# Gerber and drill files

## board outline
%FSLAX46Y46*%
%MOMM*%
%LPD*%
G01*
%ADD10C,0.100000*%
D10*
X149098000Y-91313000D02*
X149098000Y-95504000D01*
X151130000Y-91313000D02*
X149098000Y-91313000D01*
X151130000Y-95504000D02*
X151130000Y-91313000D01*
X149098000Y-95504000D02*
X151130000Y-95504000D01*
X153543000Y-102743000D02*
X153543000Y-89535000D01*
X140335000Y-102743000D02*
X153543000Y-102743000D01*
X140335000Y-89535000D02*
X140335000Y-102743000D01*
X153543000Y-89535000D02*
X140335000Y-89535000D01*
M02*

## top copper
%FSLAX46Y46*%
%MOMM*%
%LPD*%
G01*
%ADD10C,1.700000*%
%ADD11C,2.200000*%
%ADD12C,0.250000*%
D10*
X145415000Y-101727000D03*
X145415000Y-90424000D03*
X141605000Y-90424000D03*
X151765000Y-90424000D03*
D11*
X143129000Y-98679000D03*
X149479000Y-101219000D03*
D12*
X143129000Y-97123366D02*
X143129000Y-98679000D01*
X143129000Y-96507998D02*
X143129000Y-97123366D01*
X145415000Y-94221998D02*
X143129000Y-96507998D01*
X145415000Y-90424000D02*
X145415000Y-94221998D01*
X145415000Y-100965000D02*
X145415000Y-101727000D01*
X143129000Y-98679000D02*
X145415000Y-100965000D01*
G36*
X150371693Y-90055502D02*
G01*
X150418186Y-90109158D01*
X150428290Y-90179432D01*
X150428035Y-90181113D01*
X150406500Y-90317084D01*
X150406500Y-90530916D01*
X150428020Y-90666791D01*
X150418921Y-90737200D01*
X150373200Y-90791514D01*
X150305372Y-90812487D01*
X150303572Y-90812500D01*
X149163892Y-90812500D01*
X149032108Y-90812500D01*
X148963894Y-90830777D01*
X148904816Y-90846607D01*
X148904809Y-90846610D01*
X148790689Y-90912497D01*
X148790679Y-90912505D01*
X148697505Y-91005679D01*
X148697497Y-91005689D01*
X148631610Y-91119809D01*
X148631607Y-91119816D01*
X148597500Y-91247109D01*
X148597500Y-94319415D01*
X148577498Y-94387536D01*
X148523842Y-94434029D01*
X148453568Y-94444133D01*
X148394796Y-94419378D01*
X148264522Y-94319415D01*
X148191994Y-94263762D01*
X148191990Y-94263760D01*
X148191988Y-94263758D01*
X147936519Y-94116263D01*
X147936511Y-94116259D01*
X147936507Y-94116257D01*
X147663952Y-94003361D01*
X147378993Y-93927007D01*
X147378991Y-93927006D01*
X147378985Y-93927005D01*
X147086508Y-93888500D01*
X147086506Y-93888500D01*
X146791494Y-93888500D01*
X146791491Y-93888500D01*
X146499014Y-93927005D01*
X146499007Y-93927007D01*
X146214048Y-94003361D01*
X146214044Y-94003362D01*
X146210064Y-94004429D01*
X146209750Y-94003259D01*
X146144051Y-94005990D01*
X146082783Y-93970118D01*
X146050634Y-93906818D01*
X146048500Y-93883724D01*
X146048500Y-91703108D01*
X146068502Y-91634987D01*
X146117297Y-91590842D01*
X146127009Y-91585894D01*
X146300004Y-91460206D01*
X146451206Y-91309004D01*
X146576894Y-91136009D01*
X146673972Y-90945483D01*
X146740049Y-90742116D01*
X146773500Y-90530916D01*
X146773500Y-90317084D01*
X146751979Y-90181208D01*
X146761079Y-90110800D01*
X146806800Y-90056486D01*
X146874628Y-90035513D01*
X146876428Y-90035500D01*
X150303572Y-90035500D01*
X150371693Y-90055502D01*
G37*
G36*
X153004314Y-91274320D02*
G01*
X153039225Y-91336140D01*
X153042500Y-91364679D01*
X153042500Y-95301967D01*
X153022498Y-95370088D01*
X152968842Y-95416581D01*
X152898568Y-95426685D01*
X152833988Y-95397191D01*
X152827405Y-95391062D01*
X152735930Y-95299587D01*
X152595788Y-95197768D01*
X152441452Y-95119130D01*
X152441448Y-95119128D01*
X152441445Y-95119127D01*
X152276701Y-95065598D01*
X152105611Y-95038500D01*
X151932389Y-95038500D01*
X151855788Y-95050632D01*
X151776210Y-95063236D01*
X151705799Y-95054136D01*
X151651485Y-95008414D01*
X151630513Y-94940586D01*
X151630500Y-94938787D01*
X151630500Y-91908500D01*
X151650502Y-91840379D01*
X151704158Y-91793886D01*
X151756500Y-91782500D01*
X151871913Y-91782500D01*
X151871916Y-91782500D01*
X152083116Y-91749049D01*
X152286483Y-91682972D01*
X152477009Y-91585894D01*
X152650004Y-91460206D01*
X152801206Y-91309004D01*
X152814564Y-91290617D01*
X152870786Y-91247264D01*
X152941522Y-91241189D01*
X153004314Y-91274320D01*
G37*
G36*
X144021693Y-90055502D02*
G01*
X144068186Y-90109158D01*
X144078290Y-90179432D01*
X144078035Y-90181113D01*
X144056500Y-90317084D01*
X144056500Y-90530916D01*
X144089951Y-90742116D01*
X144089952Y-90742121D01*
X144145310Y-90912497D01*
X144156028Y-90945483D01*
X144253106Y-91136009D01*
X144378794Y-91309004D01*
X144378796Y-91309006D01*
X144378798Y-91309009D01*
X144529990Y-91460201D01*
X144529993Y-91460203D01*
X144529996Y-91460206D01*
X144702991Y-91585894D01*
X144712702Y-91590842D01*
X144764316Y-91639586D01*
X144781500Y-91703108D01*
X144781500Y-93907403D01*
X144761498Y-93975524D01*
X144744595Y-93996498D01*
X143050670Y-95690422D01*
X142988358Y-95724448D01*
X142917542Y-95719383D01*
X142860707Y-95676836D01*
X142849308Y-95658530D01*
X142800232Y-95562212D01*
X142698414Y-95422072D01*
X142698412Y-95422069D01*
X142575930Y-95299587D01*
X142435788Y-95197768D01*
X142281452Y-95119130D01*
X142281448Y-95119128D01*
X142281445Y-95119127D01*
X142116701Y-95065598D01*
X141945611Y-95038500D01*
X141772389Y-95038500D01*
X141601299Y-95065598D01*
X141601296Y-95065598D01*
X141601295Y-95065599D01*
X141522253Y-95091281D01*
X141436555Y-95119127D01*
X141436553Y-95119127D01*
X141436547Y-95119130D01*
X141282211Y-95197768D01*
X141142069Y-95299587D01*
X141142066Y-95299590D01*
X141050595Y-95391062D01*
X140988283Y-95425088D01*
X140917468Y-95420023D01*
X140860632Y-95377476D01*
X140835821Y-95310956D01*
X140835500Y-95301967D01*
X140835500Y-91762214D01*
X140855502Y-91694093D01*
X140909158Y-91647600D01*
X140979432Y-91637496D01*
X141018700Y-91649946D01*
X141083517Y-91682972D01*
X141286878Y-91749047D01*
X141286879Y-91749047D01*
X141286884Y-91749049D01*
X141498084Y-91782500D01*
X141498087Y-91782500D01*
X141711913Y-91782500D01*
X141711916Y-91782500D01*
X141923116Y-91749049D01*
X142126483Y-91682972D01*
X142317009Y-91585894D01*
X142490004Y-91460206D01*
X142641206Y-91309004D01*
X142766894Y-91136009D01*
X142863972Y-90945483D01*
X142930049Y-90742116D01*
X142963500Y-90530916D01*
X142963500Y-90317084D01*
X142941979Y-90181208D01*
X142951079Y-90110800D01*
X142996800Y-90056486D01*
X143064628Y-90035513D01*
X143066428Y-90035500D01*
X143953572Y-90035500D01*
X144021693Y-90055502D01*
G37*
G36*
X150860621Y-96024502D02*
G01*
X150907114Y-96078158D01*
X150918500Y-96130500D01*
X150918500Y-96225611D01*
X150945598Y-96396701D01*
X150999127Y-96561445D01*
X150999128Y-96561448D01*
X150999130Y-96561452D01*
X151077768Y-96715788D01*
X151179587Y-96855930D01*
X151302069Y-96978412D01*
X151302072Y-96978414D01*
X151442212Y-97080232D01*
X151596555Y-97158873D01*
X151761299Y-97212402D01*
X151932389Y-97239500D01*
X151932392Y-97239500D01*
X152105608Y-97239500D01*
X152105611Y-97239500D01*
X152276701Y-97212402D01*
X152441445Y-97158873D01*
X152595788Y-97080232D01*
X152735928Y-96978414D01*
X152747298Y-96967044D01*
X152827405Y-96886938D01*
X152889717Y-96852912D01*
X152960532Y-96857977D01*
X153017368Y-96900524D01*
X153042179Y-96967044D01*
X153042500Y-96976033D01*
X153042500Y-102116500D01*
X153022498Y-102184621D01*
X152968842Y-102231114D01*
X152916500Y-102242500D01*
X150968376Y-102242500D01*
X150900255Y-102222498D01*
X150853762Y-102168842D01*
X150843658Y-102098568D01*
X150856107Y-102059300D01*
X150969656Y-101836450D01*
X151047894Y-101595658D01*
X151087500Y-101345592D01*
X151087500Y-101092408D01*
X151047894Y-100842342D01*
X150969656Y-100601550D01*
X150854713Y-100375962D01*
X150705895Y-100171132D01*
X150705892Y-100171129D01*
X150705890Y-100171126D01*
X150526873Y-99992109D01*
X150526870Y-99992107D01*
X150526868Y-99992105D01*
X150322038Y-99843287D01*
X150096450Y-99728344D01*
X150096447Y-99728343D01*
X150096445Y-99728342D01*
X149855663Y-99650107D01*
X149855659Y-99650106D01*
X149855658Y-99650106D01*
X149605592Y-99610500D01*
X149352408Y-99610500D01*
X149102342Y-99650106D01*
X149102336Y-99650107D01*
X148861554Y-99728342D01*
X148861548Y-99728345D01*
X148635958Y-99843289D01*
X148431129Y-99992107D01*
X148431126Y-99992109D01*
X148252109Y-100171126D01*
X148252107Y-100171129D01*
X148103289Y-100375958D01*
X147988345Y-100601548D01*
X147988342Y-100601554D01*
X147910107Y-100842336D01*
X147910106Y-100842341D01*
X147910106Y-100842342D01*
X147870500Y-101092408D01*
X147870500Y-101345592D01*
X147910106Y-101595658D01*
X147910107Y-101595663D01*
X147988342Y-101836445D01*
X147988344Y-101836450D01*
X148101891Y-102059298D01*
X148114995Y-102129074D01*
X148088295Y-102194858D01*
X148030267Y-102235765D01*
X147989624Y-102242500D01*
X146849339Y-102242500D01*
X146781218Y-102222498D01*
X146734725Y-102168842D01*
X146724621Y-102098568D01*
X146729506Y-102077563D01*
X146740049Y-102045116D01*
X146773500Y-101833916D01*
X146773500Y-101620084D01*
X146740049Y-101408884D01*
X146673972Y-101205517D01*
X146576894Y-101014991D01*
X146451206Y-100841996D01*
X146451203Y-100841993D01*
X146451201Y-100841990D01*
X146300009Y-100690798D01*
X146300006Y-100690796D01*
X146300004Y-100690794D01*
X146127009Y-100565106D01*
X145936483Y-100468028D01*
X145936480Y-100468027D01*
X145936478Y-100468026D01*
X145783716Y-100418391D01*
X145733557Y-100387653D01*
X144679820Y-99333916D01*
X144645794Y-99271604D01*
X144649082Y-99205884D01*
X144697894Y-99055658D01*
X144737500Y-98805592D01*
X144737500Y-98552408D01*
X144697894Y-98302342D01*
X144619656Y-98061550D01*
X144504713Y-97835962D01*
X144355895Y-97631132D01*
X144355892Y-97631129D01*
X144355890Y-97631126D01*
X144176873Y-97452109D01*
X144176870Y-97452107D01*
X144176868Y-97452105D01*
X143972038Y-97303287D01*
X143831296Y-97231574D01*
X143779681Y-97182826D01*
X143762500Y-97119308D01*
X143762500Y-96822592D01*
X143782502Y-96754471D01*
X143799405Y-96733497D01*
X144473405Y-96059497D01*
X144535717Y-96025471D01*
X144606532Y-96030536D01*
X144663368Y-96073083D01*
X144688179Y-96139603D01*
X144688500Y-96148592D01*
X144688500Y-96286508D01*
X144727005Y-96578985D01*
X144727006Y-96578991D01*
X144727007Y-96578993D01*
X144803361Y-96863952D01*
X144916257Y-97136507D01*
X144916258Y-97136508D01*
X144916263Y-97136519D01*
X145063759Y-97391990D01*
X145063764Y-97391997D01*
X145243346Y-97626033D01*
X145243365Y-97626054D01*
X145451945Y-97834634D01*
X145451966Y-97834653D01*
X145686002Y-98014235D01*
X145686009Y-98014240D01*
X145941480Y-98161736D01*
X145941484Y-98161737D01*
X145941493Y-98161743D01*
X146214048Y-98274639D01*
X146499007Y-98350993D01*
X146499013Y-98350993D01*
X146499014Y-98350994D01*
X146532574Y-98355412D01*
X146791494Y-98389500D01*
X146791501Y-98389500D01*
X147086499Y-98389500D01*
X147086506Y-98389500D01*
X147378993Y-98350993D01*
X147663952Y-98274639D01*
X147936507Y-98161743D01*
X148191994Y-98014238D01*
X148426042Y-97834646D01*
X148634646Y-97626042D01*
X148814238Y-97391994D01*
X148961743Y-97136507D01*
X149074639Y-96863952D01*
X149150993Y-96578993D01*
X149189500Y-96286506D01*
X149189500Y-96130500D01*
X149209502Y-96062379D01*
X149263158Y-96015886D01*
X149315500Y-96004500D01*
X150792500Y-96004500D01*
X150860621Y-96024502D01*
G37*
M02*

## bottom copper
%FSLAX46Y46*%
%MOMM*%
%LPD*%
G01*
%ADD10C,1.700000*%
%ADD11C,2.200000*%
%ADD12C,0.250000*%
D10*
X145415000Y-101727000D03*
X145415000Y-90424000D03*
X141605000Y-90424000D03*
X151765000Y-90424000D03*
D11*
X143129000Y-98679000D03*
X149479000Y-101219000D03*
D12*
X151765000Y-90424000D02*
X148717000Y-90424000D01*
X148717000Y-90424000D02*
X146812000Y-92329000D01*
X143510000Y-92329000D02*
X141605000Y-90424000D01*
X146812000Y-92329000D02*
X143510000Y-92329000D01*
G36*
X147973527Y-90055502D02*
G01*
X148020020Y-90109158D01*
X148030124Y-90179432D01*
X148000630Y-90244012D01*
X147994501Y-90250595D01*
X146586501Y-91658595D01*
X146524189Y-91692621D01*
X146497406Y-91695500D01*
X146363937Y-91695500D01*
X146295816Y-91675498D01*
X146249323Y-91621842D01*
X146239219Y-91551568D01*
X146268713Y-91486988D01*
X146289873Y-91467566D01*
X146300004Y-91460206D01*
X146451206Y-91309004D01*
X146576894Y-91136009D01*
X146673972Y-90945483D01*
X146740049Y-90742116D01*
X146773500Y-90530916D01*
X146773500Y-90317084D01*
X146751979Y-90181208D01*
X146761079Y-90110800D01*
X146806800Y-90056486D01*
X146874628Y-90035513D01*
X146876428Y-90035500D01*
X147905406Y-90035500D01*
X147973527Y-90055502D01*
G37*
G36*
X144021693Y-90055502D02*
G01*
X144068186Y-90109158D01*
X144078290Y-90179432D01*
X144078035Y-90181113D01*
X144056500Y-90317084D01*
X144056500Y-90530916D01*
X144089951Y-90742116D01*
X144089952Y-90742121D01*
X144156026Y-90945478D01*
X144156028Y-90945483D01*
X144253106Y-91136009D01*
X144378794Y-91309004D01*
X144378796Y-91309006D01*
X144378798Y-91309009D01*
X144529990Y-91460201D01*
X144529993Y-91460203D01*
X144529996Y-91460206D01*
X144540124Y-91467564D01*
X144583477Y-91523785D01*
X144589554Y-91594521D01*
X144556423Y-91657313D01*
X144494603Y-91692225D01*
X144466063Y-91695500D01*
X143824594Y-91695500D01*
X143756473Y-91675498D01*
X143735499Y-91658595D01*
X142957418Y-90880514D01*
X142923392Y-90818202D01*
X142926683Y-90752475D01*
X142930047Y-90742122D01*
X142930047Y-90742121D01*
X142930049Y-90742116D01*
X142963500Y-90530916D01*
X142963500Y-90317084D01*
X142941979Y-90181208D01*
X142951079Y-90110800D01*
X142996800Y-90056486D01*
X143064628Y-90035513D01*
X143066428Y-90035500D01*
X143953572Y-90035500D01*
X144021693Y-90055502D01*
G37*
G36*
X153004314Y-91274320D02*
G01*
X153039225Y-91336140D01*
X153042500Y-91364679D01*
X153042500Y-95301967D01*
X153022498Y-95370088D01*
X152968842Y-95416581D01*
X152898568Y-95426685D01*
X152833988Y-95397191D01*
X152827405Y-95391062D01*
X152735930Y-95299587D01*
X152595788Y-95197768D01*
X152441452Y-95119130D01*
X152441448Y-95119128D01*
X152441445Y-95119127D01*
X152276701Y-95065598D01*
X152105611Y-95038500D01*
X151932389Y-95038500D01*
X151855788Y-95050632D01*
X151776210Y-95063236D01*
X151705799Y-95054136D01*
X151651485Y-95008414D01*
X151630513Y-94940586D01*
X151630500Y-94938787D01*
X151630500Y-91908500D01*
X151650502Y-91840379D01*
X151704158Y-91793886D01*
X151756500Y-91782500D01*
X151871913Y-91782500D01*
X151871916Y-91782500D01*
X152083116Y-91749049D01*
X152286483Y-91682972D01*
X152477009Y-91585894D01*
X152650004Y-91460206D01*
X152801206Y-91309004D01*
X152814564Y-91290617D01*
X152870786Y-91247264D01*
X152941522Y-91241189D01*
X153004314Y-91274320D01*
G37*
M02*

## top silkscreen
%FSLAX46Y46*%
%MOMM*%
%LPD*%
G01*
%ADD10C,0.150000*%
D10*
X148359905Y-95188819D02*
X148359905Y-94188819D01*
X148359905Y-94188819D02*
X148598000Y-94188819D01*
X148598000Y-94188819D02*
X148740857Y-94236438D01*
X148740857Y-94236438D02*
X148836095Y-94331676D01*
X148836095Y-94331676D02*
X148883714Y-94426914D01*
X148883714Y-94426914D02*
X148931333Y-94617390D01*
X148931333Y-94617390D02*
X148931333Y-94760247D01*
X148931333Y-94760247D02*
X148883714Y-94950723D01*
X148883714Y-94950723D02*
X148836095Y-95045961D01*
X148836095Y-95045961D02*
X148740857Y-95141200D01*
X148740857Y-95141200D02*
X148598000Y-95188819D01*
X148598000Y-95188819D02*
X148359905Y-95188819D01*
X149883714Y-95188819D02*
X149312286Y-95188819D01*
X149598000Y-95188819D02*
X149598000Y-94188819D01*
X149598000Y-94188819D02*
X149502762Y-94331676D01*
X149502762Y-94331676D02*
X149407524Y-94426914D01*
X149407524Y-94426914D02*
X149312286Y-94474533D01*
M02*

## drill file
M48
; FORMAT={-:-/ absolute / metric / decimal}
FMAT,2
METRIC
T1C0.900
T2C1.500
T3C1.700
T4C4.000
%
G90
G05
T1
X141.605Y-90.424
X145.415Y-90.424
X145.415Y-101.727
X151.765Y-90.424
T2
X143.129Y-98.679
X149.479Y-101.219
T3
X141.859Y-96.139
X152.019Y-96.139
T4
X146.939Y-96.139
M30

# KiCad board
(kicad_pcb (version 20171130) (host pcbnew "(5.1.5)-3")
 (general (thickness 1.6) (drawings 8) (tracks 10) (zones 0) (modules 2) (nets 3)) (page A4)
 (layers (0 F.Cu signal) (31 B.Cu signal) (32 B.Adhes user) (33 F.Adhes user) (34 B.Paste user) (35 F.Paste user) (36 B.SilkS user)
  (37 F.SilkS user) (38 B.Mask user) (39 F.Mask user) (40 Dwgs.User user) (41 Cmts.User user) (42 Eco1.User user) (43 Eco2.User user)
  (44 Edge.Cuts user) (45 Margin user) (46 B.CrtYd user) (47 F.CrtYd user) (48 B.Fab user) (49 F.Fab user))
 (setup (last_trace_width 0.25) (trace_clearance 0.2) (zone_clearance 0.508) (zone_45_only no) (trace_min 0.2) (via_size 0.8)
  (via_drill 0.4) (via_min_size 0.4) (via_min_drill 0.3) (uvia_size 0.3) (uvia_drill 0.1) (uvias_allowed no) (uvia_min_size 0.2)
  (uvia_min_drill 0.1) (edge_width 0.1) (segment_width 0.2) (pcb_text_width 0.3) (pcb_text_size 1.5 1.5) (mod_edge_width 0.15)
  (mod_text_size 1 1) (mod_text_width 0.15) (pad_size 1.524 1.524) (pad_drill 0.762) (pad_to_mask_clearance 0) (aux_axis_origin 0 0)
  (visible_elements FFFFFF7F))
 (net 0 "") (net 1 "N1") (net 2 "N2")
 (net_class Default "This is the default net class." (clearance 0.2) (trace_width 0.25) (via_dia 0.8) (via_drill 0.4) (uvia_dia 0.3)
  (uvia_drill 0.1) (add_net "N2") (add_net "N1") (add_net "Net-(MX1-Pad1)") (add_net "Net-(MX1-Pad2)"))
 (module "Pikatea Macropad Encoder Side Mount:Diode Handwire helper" (layer F.Cu) (at 149.098 94.234)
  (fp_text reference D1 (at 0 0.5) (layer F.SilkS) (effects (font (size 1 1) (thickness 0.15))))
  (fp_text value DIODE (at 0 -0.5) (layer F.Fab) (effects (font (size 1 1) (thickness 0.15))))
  (pad 2 thru_hole circle (at -3.683 7.493 90) (size 1.7 1.7) (drill 0.9) (layers *.Cu *.Mask) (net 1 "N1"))
  (pad 2 thru_hole circle (at -3.683 -3.81 90) (size 1.7 1.7) (drill 0.9) (layers *.Cu *.Mask) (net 1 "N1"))
  (pad 1 thru_hole circle (at -7.493 -3.81 90) (size 1.7 1.7) (drill 0.9) (layers *.Cu *.Mask) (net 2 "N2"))
  (pad 1 thru_hole circle (at 2.667 -3.81 90) (size 1.7 1.7) (drill 0.9) (layers *.Cu *.Mask) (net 2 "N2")))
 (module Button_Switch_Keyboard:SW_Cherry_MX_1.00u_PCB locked (layer B.Cu) (at 149.479 101.219)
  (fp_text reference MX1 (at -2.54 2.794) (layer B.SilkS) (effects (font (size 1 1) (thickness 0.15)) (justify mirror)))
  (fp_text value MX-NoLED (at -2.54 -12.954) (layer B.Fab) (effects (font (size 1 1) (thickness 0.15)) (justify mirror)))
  (pad "" np_thru_hole circle (at 2.54 -5.08) (size 1.7 1.7) (drill 1.7) (layers *.Cu *.Mask))
  (pad "" np_thru_hole circle (at -7.62 -5.08) (size 1.7 1.7) (drill 1.7) (layers *.Cu *.Mask))
  (pad "" np_thru_hole circle (at -2.54 -5.08) (size 4 4) (drill 4) (layers *.Cu *.Mask))
  (pad 2 thru_hole circle (at -6.35 -2.54) (size 2.2 2.2) (drill 1.5) (layers *.Cu *.Mask) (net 1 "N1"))
  (pad 1 thru_hole circle (at 0 0) (size 2.2 2.2) (drill 1.5) (layers *.Cu *.Mask)))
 (gr_line (start 149.098 91.313) (end 149.098 95.504) (layer Edge.Cuts) (width 0.1))
 (gr_line (start 151.13 91.313) (end 149.098 91.313) (layer Edge.Cuts) (width 0.1))
 (gr_line (start 151.13 95.504) (end 151.13 91.313) (layer Edge.Cuts) (width 0.1))
 (gr_line (start 149.098 95.504) (end 151.13 95.504) (layer Edge.Cuts) (width 0.1))
 (gr_line (start 153.543 102.743) (end 153.543 89.535) (layer Edge.Cuts) (width 0.1))
 (gr_line (start 140.335 102.743) (end 153.543 102.743) (layer Edge.Cuts) (width 0.1))
 (gr_line (start 140.335 89.535) (end 140.335 102.743) (layer Edge.Cuts) (width 0.1))
 (gr_line (start 153.543 89.535) (end 140.335 89.535) (layer Edge.Cuts) (width 0.1))
 (segment (start 143.129 97.123366) (end 143.129 98.679) (width 0.25) (layer F.Cu) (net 1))
 (segment (start 143.129 96.507998) (end 143.129 97.123366) (width 0.25) (layer F.Cu) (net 1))
 (segment (start 145.415 94.221998) (end 143.129 96.507998) (width 0.25) (layer F.Cu) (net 1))
 (segment (start 145.415 90.424) (end 145.415 94.221998) (width 0.25) (layer F.Cu) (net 1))
 (segment (start 145.415 100.965) (end 145.415 101.727) (width 0.25) (layer F.Cu) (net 1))
 (segment (start 143.129 98.679) (end 145.415 100.965) (width 0.25) (layer F.Cu) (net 1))
 (segment (start 151.765 90.424) (end 148.717 90.424) (width 0.25) (layer B.Cu) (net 2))
 (segment (start 148.717 90.424) (end 146.812 92.329) (width 0.25) (layer B.Cu) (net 2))
 (segment (start 143.51 92.329) (end 141.605 90.424) (width 0.25) (layer B.Cu) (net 2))
 (segment (start 146.812 92.329) (end 143.51 92.329) (width 0.25) (layer B.Cu) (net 2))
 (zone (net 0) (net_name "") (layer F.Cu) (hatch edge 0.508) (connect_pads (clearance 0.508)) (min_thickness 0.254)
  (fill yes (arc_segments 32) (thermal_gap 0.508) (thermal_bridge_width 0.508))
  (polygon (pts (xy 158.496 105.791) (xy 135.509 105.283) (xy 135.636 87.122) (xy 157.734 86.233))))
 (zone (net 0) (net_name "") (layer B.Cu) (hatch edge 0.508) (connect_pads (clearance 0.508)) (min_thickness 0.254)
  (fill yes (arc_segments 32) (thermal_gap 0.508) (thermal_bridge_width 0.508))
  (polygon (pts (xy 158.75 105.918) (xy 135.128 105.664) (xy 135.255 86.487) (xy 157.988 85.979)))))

